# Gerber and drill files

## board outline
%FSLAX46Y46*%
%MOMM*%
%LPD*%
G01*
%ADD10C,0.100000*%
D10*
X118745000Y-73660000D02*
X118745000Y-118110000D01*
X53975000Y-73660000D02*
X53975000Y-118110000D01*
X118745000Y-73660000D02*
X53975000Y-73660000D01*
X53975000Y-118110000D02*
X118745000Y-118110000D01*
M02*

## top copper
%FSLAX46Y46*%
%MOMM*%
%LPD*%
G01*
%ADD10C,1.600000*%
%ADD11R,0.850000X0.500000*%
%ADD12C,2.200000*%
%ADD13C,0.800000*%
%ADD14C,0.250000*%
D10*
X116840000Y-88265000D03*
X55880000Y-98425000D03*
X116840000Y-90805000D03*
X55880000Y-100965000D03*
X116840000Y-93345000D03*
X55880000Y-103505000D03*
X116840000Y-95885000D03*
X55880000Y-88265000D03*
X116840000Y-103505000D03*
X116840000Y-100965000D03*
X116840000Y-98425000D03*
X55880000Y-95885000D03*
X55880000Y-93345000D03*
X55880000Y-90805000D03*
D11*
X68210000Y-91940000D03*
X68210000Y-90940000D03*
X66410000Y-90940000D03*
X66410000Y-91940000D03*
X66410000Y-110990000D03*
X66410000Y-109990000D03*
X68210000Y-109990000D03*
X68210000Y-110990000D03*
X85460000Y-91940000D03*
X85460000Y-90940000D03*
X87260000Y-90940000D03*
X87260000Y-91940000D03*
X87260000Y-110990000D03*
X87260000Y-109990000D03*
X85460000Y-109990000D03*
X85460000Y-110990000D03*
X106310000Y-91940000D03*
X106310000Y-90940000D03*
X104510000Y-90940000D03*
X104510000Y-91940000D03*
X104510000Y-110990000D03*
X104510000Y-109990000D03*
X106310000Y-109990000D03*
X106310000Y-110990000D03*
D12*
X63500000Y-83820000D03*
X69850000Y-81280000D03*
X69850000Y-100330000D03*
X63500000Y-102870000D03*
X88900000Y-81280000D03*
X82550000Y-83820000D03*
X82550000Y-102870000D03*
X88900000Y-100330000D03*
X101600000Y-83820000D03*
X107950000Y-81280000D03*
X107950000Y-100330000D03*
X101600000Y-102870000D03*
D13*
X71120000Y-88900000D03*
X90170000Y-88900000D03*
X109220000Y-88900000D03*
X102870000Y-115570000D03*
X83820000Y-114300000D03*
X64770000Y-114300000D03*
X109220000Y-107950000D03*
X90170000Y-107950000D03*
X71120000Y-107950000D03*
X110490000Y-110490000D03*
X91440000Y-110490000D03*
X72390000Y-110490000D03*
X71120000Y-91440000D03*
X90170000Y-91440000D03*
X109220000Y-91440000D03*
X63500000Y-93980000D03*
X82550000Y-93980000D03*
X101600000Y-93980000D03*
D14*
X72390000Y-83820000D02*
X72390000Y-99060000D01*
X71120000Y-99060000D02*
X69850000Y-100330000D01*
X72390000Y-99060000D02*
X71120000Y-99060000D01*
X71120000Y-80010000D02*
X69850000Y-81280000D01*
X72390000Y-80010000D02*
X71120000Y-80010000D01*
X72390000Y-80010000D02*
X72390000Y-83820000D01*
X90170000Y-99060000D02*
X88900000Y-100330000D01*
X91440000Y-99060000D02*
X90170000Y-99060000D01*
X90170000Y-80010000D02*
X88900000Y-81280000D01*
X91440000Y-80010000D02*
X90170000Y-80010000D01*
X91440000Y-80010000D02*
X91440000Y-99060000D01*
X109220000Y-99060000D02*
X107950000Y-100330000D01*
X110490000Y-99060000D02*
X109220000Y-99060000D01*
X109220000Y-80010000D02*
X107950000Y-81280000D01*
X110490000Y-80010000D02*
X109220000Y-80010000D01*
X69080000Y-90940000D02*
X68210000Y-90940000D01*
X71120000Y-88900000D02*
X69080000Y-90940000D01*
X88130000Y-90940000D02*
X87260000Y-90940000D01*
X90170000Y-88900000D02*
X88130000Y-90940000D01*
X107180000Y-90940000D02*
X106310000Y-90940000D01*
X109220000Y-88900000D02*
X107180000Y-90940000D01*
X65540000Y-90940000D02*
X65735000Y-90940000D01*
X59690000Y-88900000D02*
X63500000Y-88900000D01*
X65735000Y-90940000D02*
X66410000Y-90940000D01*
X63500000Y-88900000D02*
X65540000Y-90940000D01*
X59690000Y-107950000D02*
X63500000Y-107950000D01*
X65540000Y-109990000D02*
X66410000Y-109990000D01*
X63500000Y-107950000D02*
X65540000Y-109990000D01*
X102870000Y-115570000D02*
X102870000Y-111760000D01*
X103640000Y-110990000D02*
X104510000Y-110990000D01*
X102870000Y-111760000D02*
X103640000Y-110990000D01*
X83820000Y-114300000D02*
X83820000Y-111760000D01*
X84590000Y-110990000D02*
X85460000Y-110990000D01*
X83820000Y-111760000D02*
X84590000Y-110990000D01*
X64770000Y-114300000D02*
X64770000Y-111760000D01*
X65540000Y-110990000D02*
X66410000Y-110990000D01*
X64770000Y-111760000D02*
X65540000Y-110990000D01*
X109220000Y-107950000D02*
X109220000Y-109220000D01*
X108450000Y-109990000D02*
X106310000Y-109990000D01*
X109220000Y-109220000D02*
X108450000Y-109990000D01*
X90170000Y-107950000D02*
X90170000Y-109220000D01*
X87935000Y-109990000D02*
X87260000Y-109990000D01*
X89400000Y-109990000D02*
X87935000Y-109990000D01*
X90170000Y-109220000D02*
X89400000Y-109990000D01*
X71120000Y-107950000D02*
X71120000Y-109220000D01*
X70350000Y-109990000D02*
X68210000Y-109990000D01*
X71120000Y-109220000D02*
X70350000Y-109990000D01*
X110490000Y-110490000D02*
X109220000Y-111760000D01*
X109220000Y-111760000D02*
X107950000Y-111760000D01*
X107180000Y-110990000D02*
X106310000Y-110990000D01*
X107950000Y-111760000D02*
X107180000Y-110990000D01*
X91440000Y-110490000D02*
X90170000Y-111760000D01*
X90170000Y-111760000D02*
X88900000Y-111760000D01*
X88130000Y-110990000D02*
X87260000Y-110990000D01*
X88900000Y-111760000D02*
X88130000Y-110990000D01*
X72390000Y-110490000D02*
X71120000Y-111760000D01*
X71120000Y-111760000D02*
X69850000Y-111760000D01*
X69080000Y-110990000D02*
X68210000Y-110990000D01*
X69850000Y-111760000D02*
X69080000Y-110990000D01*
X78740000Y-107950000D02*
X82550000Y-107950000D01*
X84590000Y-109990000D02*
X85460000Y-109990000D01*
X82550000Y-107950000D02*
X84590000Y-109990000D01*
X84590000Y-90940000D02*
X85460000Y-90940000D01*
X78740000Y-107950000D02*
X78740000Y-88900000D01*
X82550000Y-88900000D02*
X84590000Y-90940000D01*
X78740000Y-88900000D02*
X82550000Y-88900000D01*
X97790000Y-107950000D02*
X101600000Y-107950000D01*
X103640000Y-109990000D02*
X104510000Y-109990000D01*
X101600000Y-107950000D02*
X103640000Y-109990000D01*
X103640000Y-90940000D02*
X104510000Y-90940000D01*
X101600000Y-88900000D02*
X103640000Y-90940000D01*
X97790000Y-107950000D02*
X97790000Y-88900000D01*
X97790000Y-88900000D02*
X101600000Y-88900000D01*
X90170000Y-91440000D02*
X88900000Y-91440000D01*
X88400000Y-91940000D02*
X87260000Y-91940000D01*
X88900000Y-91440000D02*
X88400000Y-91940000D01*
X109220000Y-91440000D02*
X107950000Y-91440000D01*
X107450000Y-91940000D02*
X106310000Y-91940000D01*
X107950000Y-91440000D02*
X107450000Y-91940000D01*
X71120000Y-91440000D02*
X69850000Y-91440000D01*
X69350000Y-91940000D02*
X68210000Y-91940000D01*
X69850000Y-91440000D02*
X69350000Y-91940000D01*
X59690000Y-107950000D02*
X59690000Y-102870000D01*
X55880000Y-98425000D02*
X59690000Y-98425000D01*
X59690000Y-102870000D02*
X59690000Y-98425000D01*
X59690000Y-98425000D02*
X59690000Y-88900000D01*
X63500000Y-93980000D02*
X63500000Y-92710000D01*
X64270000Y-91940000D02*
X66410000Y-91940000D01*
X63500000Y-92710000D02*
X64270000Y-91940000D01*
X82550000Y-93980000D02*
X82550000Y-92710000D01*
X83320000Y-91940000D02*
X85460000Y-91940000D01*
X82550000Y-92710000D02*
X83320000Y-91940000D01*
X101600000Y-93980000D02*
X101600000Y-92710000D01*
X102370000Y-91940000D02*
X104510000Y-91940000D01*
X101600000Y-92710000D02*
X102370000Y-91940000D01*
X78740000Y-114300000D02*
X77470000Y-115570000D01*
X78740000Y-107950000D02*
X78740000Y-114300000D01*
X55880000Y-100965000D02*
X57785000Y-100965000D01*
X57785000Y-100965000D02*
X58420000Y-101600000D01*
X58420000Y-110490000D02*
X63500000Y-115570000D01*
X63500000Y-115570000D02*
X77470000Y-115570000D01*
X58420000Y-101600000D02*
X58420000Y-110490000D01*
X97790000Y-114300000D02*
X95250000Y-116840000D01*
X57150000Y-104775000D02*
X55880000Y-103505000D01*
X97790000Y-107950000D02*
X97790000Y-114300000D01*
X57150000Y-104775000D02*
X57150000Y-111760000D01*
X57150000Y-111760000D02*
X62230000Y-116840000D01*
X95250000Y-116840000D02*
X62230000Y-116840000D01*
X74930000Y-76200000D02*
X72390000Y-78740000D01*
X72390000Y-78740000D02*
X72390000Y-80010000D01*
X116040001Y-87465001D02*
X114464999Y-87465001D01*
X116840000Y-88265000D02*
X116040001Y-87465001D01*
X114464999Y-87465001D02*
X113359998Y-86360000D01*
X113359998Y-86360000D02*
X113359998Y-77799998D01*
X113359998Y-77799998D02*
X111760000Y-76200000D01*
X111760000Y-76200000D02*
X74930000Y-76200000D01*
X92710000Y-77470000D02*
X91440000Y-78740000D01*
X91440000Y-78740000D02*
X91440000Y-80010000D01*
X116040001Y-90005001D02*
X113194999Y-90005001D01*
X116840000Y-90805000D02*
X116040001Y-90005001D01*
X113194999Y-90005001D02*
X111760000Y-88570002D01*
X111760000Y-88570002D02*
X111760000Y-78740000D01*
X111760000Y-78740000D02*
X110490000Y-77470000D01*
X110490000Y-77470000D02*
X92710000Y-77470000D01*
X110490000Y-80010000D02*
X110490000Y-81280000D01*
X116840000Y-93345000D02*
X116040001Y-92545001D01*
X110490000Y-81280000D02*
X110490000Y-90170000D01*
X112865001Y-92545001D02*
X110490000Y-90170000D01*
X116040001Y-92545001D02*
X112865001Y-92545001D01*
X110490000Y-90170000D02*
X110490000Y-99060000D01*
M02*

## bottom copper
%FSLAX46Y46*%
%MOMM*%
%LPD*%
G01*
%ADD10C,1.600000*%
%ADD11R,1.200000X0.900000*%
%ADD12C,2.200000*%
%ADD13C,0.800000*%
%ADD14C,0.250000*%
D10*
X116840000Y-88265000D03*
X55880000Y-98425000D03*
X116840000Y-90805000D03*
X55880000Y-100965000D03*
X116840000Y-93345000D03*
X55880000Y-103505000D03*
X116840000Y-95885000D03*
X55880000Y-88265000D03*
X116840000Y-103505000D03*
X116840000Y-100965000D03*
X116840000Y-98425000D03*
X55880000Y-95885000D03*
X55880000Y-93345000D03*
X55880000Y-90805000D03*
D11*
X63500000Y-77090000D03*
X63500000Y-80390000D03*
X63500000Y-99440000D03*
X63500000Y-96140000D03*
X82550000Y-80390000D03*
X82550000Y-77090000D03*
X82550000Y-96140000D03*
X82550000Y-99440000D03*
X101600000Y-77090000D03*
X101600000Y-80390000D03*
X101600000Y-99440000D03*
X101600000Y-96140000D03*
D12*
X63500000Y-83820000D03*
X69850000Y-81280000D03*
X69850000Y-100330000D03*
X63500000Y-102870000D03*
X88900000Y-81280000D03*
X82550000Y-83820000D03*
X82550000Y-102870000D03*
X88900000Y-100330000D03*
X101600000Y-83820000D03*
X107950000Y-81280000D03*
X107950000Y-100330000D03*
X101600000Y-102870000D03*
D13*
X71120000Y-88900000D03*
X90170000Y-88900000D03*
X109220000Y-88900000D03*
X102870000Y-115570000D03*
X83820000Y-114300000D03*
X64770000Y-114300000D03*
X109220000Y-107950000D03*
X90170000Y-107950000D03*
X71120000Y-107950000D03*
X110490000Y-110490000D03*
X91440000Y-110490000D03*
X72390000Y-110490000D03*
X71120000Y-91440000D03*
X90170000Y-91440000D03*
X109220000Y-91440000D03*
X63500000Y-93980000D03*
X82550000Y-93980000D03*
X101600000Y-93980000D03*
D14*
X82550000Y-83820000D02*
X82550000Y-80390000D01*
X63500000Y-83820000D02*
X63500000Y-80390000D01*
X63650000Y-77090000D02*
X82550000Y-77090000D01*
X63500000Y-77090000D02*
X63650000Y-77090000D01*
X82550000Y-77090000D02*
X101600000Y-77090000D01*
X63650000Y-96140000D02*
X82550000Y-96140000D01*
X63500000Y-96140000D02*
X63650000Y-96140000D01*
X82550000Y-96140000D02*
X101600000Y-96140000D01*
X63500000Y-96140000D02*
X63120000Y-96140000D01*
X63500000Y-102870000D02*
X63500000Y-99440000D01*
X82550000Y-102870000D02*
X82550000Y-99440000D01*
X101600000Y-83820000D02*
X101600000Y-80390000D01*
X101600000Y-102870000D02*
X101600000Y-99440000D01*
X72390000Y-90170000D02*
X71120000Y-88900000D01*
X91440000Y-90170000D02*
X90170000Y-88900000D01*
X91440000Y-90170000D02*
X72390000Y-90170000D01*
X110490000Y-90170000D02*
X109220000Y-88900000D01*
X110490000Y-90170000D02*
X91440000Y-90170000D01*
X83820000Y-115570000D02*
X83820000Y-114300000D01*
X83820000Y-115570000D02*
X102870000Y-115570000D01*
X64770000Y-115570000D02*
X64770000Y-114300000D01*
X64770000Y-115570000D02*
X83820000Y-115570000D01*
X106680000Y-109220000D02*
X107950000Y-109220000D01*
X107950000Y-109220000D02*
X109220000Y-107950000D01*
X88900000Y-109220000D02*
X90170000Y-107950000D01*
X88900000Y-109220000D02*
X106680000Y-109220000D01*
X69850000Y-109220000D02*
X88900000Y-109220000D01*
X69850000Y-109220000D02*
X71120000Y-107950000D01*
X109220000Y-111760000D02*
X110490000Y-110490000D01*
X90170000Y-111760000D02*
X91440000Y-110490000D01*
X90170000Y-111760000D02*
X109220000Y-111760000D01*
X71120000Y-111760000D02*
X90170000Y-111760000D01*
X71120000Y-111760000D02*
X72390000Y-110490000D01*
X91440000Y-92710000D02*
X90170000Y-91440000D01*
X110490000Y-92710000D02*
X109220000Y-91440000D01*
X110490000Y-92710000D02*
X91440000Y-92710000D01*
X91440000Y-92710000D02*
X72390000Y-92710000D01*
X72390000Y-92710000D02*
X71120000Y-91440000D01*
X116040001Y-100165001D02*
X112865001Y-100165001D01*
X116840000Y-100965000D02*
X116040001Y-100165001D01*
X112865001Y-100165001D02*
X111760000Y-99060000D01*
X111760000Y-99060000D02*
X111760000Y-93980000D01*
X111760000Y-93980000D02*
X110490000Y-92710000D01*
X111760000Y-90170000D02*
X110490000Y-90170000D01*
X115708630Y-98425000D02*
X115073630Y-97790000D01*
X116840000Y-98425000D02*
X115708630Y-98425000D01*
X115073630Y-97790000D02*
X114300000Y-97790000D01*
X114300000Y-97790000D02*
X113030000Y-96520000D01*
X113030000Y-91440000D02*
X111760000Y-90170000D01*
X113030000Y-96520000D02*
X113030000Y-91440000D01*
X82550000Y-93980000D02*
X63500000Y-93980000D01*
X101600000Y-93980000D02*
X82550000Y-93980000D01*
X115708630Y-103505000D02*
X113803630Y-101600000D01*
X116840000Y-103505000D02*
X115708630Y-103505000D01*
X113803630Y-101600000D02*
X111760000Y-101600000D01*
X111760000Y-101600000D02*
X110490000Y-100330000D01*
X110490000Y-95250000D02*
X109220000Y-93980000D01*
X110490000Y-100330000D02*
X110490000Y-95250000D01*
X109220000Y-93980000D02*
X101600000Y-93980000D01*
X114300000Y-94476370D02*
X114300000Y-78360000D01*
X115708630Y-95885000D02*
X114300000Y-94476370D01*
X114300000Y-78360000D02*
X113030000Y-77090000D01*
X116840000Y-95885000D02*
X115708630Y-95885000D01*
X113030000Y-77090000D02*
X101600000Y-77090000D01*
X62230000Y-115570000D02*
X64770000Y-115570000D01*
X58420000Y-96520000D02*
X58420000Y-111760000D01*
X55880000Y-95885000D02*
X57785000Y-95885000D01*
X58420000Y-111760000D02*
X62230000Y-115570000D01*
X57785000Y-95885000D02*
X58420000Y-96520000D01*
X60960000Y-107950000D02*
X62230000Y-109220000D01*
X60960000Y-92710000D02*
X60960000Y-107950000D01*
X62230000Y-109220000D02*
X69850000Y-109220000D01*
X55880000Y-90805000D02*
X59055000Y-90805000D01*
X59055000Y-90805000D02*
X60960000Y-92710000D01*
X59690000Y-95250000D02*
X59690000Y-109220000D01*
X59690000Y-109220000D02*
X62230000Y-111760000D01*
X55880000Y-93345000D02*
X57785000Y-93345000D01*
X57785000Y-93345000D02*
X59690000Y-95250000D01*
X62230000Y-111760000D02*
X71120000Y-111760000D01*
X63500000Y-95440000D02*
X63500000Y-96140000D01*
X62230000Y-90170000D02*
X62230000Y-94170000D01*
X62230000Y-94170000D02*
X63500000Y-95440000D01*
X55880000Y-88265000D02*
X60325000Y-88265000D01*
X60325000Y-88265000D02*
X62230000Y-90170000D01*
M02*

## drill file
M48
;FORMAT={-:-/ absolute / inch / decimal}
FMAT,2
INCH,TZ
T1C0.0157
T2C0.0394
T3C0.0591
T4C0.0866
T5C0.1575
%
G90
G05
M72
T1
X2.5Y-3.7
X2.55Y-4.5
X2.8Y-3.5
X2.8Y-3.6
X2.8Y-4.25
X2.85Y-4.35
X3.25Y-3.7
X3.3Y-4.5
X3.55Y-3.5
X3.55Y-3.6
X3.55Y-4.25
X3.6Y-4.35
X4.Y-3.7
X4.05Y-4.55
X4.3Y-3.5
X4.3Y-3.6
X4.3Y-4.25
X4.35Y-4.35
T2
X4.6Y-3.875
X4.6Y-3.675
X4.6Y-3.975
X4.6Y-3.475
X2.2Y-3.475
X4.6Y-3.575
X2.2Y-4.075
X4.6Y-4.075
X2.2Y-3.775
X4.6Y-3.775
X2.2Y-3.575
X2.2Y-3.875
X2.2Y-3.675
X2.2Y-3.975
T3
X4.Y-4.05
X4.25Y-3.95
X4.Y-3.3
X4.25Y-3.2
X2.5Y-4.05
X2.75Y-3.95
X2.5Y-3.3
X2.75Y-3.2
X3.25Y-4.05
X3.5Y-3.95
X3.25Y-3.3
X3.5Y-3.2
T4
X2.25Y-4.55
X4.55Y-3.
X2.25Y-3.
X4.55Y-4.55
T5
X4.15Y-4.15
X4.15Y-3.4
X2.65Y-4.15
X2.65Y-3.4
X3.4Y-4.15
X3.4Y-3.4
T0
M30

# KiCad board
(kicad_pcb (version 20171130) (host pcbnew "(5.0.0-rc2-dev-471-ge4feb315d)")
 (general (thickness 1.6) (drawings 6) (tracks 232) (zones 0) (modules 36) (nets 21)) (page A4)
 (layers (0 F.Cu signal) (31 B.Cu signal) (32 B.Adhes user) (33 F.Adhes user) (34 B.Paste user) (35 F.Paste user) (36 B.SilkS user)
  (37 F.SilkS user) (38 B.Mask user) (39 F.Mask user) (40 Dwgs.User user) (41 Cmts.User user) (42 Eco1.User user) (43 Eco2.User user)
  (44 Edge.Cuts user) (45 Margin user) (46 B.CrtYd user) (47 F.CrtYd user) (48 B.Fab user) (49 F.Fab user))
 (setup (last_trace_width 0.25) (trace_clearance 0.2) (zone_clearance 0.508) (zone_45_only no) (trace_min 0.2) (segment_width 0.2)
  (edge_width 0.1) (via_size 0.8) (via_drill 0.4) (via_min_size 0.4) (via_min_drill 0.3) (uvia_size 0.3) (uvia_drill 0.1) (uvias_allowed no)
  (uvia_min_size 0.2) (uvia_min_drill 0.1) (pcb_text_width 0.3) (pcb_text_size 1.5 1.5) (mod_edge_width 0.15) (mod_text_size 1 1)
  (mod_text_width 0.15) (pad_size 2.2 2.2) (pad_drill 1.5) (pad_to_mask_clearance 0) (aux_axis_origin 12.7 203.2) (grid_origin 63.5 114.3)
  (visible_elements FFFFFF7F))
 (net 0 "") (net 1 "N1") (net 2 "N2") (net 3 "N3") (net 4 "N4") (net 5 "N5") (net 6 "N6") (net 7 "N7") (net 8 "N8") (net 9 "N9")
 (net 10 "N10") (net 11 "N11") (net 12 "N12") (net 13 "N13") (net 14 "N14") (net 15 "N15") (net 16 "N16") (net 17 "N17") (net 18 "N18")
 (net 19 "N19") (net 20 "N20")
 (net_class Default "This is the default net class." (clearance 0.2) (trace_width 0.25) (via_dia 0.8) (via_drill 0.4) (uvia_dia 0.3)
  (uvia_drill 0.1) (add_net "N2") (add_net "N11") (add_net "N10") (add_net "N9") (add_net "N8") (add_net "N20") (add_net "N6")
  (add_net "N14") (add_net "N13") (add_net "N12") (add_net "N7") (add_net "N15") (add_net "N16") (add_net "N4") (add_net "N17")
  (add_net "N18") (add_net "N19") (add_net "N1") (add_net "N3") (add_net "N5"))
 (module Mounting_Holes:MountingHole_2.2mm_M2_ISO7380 (layer F.Cu) (at 115.57 76.2)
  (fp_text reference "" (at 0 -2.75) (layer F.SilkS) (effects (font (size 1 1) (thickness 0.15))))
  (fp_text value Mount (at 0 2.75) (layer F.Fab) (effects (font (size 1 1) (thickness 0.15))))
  (pad 1 np_thru_hole circle (at 0 0) (size 2.2 2.2) (drill 2.2) (layers *.Cu *.Mask)))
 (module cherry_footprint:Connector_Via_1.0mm (layer F.Cu) (at 116.84 88.265 90)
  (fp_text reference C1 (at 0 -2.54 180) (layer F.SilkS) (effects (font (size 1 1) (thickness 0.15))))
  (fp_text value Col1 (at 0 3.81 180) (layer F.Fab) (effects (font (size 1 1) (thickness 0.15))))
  (pad 1 thru_hole circle (at 0 0 90) (size 1.6 1.6) (drill 1) (layers *.Cu *.Mask) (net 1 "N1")))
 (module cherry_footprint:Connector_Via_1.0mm (layer F.Cu) (at 55.88 98.425 270)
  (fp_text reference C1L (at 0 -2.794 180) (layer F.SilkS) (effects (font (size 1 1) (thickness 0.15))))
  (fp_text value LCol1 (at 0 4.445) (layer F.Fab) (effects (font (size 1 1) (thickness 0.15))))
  (pad 1 thru_hole circle (at 0 0 270) (size 1.6 1.6) (drill 1) (layers *.Cu *.Mask) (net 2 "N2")))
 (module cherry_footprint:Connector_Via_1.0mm (layer F.Cu) (at 116.84 90.805 90)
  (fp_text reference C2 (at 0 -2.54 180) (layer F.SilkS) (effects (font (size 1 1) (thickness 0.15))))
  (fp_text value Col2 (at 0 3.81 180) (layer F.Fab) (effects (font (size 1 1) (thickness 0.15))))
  (pad 1 thru_hole circle (at 0 0 90) (size 1.6 1.6) (drill 1) (layers *.Cu *.Mask) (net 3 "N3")))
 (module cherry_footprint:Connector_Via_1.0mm (layer F.Cu) (at 55.88 100.965 270)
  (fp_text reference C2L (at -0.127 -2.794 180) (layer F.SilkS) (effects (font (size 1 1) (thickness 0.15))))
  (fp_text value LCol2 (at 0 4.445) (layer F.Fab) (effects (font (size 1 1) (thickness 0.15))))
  (pad 1 thru_hole circle (at 0 0 270) (size 1.6 1.6) (drill 1) (layers *.Cu *.Mask) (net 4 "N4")))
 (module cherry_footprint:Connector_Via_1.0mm (layer F.Cu) (at 116.84 93.345 90)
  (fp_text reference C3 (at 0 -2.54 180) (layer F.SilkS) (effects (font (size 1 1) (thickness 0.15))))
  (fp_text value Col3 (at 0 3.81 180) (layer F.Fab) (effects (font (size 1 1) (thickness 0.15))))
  (pad 1 thru_hole circle (at 0 0 90) (size 1.6 1.6) (drill 1) (layers *.Cu *.Mask) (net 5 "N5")))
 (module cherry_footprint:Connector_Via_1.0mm (layer F.Cu) (at 55.88 103.505 270)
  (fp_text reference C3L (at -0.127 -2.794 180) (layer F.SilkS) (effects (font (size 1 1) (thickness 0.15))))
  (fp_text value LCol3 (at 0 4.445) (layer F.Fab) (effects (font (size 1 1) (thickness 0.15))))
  (pad 1 thru_hole circle (at 0 0 270) (size 1.6 1.6) (drill 1) (layers *.Cu *.Mask) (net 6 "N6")))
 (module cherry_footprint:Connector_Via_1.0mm (layer F.Cu) (at 116.84 95.885 90)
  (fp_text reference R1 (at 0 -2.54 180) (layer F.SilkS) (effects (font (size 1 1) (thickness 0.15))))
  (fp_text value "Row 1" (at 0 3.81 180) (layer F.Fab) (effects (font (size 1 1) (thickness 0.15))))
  (pad 1 thru_hole circle (at 0 0 90) (size 1.6 1.6) (drill 1) (layers *.Cu *.Mask) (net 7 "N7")))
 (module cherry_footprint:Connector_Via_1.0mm (layer F.Cu) (at 55.88 88.265 270)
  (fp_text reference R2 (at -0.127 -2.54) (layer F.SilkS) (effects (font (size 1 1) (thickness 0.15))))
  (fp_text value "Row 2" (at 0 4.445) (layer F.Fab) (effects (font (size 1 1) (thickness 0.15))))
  (pad 1 thru_hole circle (at 0 0 270) (size 1.6 1.6) (drill 1) (layers *.Cu *.Mask) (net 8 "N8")))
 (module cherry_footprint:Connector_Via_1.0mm (layer F.Cu) (at 116.84 103.505 90)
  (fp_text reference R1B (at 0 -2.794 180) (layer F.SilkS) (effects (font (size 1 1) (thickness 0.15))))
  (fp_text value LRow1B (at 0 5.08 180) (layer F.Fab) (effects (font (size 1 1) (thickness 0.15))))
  (pad 1 thru_hole circle (at 0 0 90) (size 1.6 1.6) (drill 1) (layers *.Cu *.Mask) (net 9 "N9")))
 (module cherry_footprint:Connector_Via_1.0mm (layer F.Cu) (at 116.84 100.965 90)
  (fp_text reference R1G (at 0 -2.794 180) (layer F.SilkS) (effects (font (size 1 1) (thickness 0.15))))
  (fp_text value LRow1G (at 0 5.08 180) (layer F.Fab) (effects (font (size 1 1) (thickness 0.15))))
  (pad 1 thru_hole circle (at 0 0 90) (size 1.6 1.6) (drill 1) (layers *.Cu *.Mask) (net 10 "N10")))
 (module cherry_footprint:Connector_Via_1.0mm (layer F.Cu) (at 116.84 98.425 90)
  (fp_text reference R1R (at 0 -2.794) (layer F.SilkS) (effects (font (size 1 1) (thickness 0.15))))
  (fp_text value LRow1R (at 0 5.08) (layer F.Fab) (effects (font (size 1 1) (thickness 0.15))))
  (pad 1 thru_hole circle (at 0 0 90) (size 1.6 1.6) (drill 1) (layers *.Cu *.Mask) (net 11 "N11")))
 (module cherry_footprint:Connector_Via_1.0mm (layer F.Cu) (at 55.88 95.885 270)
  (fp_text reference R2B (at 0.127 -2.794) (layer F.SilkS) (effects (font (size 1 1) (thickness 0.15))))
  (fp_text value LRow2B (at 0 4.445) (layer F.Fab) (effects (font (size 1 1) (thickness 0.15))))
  (pad 1 thru_hole circle (at 0 0 270) (size 1.6 1.6) (drill 1) (layers *.Cu *.Mask) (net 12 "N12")))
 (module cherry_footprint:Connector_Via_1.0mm (layer F.Cu) (at 55.88 93.345 270)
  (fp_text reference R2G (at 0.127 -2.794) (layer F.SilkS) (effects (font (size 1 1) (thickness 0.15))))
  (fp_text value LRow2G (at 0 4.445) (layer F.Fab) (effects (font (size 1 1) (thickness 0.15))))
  (pad 1 thru_hole circle (at 0 0 270) (size 1.6 1.6) (drill 1) (layers *.Cu *.Mask) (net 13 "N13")))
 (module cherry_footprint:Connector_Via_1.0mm (layer F.Cu) (at 55.88 90.805 270)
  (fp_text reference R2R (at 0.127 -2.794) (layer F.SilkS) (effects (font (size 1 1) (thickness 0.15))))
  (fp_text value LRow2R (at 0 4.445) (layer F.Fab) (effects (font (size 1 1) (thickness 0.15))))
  (pad 1 thru_hole circle (at 0 0 270) (size 1.6 1.6) (drill 1) (layers *.Cu *.Mask) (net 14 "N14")))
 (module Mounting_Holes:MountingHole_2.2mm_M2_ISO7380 (layer F.Cu) (at 57.15 115.57)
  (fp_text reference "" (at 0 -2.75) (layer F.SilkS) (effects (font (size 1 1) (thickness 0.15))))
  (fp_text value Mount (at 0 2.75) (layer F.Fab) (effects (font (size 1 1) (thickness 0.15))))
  (pad 1 np_thru_hole circle (at 0 0) (size 2.2 2.2) (drill 2.2) (layers *.Cu *.Mask)))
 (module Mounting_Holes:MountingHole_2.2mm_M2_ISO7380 (layer F.Cu) (at 115.57 115.57)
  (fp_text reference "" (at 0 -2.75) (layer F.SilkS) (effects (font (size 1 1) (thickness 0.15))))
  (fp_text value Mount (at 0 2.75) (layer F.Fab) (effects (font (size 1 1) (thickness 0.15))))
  (pad 1 np_thru_hole circle (at 0 0) (size 2.2 2.2) (drill 2.2) (layers *.Cu *.Mask)))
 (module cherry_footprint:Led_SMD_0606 (layer F.Cu) (at 67.31 91.44 180)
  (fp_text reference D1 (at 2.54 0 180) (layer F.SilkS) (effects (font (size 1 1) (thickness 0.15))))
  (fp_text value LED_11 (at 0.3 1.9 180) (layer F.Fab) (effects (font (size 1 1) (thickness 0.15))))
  (pad 3 smd rect (at -0.9 -0.5 180) (size 0.85 0.5) (layers F.Cu F.Paste F.Mask) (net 10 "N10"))
  (pad 2 smd rect (at -0.9 0.5 180) (size 0.85 0.5) (layers F.Cu F.Paste F.Mask) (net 11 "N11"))
  (pad 1 smd rect (at 0.9 0.5 180) (size 0.85 0.5) (layers F.Cu F.Paste F.Mask) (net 2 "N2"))
  (pad 4 smd rect (at 0.9 -0.5 180) (size 0.85 0.5) (layers F.Cu F.Paste F.Mask) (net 9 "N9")))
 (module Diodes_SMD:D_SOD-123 (layer B.Cu) (at 63.5 78.74 270)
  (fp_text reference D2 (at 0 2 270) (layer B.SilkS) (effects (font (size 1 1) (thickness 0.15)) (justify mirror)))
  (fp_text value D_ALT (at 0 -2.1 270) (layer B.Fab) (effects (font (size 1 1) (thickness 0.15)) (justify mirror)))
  (pad 1 smd rect (at -1.65 0 270) (size 0.9 1.2) (layers B.Cu B.Paste B.Mask) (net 7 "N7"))
  (pad 2 smd rect (at 1.65 0 270) (size 0.9 1.2) (layers B.Cu B.Paste B.Mask) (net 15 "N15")))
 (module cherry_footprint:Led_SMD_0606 (layer F.Cu) (at 67.31 110.49 180)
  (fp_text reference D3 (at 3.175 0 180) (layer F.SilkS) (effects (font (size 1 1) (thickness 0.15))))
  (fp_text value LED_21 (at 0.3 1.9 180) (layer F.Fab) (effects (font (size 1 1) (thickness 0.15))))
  (pad 4 smd rect (at 0.9 -0.5 180) (size 0.85 0.5) (layers F.Cu F.Paste F.Mask) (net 12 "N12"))
  (pad 1 smd rect (at 0.9 0.5 180) (size 0.85 0.5) (layers F.Cu F.Paste F.Mask) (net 2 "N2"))
  (pad 2 smd rect (at -0.9 0.5 180) (size 0.85 0.5) (layers F.Cu F.Paste F.Mask) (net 14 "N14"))
  (pad 3 smd rect (at -0.9 -0.5 180) (size 0.85 0.5) (layers F.Cu F.Paste F.Mask) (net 13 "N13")))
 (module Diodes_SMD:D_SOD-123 (layer B.Cu) (at 63.5 97.79 270)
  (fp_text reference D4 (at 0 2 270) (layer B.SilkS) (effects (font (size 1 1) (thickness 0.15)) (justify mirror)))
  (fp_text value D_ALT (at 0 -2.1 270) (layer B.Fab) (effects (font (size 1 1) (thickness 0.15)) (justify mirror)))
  (pad 2 smd rect (at 1.65 0 270) (size 0.9 1.2) (layers B.Cu B.Paste B.Mask) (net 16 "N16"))
  (pad 1 smd rect (at -1.65 0 270) (size 0.9 1.2) (layers B.Cu B.Paste B.Mask) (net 8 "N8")))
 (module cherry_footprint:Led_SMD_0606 (layer F.Cu) (at 86.36 91.44 180)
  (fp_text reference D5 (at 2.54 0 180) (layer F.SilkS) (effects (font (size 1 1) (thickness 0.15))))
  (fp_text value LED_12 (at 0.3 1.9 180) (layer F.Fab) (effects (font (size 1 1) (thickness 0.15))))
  (pad 4 smd rect (at 0.9 -0.5 180) (size 0.85 0.5) (layers F.Cu F.Paste F.Mask) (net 9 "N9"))
  (pad 1 smd rect (at 0.9 0.5 180) (size 0.85 0.5) (layers F.Cu F.Paste F.Mask) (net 4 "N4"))
  (pad 2 smd rect (at -0.9 0.5 180) (size 0.85 0.5) (layers F.Cu F.Paste F.Mask) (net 11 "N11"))
  (pad 3 smd rect (at -0.9 -0.5 180) (size 0.85 0.5) (layers F.Cu F.Paste F.Mask) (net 10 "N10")))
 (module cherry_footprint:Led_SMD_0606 (layer F.Cu) (at 86.36 110.49 180)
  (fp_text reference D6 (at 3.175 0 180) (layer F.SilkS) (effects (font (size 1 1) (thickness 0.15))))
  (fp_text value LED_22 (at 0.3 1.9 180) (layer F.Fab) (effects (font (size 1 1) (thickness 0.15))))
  (pad 3 smd rect (at -0.9 -0.5 180) (size 0.85 0.5) (layers F.Cu F.Paste F.Mask) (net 13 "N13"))
  (pad 2 smd rect (at -0.9 0.5 180) (size 0.85 0.5) (layers F.Cu F.Paste F.Mask) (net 14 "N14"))
  (pad 1 smd rect (at 0.9 0.5 180) (size 0.85 0.5) (layers F.Cu F.Paste F.Mask) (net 4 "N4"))
  (pad 4 smd rect (at 0.9 -0.5 180) (size 0.85 0.5) (layers F.Cu F.Paste F.Mask) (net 12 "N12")))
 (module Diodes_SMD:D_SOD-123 (layer B.Cu) (at 82.55 78.74 270)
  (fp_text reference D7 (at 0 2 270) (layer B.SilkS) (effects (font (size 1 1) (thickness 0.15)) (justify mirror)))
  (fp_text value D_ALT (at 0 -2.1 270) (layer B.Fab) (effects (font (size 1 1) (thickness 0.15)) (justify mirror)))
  (pad 2 smd rect (at 1.65 0 270) (size 0.9 1.2) (layers B.Cu B.Paste B.Mask) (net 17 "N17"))
  (pad 1 smd rect (at -1.65 0 270) (size 0.9 1.2) (layers B.Cu B.Paste B.Mask) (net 7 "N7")))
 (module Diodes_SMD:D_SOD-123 (layer B.Cu) (at 82.55 97.79 270)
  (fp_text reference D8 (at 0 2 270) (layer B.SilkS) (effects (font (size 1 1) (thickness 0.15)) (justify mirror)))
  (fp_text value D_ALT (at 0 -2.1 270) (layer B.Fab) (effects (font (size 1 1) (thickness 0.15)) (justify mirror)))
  (pad 1 smd rect (at -1.65 0 270) (size 0.9 1.2) (layers B.Cu B.Paste B.Mask) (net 8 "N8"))
  (pad 2 smd rect (at 1.65 0 270) (size 0.9 1.2) (layers B.Cu B.Paste B.Mask) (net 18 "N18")))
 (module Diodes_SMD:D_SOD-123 (layer B.Cu) (at 101.6 78.74 270)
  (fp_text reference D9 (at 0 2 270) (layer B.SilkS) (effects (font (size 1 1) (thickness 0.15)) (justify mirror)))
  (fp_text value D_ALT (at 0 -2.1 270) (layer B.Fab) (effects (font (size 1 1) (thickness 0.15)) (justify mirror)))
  (pad 1 smd rect (at -1.65 0 270) (size 0.9 1.2) (layers B.Cu B.Paste B.Mask) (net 7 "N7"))
  (pad 2 smd rect (at 1.65 0 270) (size 0.9 1.2) (layers B.Cu B.Paste B.Mask) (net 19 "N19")))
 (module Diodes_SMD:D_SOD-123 (layer B.Cu) (at 101.6 97.79 270)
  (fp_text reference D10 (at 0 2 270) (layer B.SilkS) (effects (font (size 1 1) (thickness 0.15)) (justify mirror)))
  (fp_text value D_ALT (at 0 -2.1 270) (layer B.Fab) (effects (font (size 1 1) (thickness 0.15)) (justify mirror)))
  (pad 2 smd rect (at 1.65 0 270) (size 0.9 1.2) (layers B.Cu B.Paste B.Mask) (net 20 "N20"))
  (pad 1 smd rect (at -1.65 0 270) (size 0.9 1.2) (layers B.Cu B.Paste B.Mask) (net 8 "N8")))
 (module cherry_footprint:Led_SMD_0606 (layer F.Cu) (at 105.41 91.44 180)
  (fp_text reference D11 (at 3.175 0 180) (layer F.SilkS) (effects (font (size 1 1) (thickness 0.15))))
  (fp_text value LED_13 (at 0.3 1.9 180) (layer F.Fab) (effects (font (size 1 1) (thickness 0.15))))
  (pad 3 smd rect (at -0.9 -0.5 180) (size 0.85 0.5) (layers F.Cu F.Paste F.Mask) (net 10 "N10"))
  (pad 2 smd rect (at -0.9 0.5 180) (size 0.85 0.5) (layers F.Cu F.Paste F.Mask) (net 11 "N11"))
  (pad 1 smd rect (at 0.9 0.5 180) (size 0.85 0.5) (layers F.Cu F.Paste F.Mask) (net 6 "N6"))
  (pad 4 smd rect (at 0.9 -0.5 180) (size 0.85 0.5) (layers F.Cu F.Paste F.Mask) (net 9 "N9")))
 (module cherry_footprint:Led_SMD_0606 (layer F.Cu) (at 105.41 110.49 180)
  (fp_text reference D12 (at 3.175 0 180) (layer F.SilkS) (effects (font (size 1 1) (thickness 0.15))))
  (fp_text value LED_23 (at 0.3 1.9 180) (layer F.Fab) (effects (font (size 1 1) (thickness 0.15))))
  (pad 4 smd rect (at 0.9 -0.5 180) (size 0.85 0.5) (layers F.Cu F.Paste F.Mask) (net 12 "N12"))
  (pad 1 smd rect (at 0.9 0.5 180) (size 0.85 0.5) (layers F.Cu F.Paste F.Mask) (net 6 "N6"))
  (pad 2 smd rect (at -0.9 0.5 180) (size 0.85 0.5) (layers F.Cu F.Paste F.Mask) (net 14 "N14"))
  (pad 3 smd rect (at -0.9 -0.5 180) (size 0.85 0.5) (layers F.Cu F.Paste F.Mask) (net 13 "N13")))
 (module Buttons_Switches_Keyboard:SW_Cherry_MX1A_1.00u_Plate (layer F.Cu) (at 69.85 81.28)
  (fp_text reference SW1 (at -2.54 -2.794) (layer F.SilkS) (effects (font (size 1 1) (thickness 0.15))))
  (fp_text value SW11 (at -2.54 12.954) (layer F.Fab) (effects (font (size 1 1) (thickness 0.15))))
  (pad "" np_thru_hole circle (at -2.54 5.08) (size 4 4) (drill 4) (layers *.Cu *.Mask))
  (pad 2 thru_hole circle (at -6.35 2.54) (size 2.2 2.2) (drill 1.5) (layers *.Cu *.Mask) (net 15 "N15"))
  (pad 1 thru_hole circle (at 0 0) (size 2.2 2.2) (drill 1.5) (layers *.Cu *.Mask) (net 1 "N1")))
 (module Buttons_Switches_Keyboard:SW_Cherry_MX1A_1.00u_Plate (layer F.Cu) (at 69.85 100.33)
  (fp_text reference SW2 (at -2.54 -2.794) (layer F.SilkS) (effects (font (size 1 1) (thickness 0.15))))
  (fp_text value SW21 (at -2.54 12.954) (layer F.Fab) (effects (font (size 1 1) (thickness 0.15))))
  (pad 1 thru_hole circle (at 0 0) (size 2.2 2.2) (drill 1.5) (layers *.Cu *.Mask) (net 1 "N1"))
  (pad 2 thru_hole circle (at -6.35 2.54) (size 2.2 2.2) (drill 1.5) (layers *.Cu *.Mask) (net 16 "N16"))
  (pad "" np_thru_hole circle (at -2.54 5.08) (size 4 4) (drill 4) (layers *.Cu *.Mask)))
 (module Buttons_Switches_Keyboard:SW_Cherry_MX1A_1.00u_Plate (layer F.Cu) (at 88.9 81.28)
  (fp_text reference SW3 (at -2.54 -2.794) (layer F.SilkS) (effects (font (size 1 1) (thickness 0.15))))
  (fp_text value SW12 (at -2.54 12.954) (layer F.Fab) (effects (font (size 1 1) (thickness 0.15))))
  (pad 1 thru_hole circle (at 0 0) (size 2.2 2.2) (drill 1.5) (layers *.Cu *.Mask) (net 3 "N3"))
  (pad 2 thru_hole circle (at -6.35 2.54) (size 2.2 2.2) (drill 1.5) (layers *.Cu *.Mask) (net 17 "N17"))
  (pad "" np_thru_hole circle (at -2.54 5.08) (size 4 4) (drill 4) (layers *.Cu *.Mask)))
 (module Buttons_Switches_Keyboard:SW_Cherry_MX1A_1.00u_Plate (layer F.Cu) (at 88.9 100.33)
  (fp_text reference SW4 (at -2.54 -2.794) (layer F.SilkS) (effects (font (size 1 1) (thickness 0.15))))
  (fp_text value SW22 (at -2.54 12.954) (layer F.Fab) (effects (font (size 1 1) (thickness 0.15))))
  (pad "" np_thru_hole circle (at -2.54 5.08) (size 4 4) (drill 4) (layers *.Cu *.Mask))
  (pad 2 thru_hole circle (at -6.35 2.54) (size 2.2 2.2) (drill 1.5) (layers *.Cu *.Mask) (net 18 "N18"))
  (pad 1 thru_hole circle (at 0 0) (size 2.2 2.2) (drill 1.5) (layers *.Cu *.Mask) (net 3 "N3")))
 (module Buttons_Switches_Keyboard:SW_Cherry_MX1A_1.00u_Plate (layer F.Cu) (at 107.95 81.28)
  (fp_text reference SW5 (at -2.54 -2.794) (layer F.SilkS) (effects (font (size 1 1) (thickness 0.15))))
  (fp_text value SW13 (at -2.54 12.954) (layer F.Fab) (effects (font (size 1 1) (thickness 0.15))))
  (pad "" np_thru_hole circle (at -2.54 5.08) (size 4 4) (drill 4) (layers *.Cu *.Mask))
  (pad 2 thru_hole circle (at -6.35 2.54) (size 2.2 2.2) (drill 1.5) (layers *.Cu *.Mask) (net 19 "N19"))
  (pad 1 thru_hole circle (at 0 0) (size 2.2 2.2) (drill 1.5) (layers *.Cu *.Mask) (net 5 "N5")))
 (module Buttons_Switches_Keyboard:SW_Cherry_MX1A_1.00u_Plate (layer F.Cu) (at 107.95 100.33)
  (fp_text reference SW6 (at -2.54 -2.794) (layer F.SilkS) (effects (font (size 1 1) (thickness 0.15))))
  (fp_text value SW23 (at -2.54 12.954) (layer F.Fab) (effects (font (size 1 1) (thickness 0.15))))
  (pad 1 thru_hole circle (at 0 0) (size 2.2 2.2) (drill 1.5) (layers *.Cu *.Mask) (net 5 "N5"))
  (pad 2 thru_hole circle (at -6.35 2.54) (size 2.2 2.2) (drill 1.5) (layers *.Cu *.Mask) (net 20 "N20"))
  (pad "" np_thru_hole circle (at -2.54 5.08) (size 4 4) (drill 4) (layers *.Cu *.Mask)))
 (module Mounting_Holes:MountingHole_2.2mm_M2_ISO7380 (layer F.Cu) (at 57.15 76.2)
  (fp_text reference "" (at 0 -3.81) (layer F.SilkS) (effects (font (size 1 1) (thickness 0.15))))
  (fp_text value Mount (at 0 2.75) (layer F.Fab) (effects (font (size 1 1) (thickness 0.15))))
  (pad 1 np_thru_hole circle (at 0 0) (size 2.2 2.2) (drill 2.2) (layers *.Cu *.Mask)))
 (gr_line (start 118.745 73.66) (end 118.745 118.11) (layer Edge.Cuts) (width 0.1))
 (gr_line (start 53.975 73.66) (end 53.975 118.11) (layer Edge.Cuts) (width 0.1))
 (gr_line (start 118.745 73.66) (end 53.975 73.66) (layer Edge.Cuts) (width 0.1))
 (gr_line (start 53.975 118.11) (end 118.745 118.11) (layer Edge.Cuts) (width 0.1))
 (segment (start 72.39 83.82) (end 72.39 99.06) (width 0.25) (layer F.Cu) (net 1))
 (segment (start 71.12 99.06) (end 69.85 100.33) (width 0.25) (layer F.Cu) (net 1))
 (segment (start 72.39 99.06) (end 71.12 99.06) (width 0.25) (layer F.Cu) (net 1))
 (segment (start 71.12 80.01) (end 69.85 81.28) (width 0.25) (layer F.Cu) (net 1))
 (segment (start 72.39 80.01) (end 71.12 80.01) (width 0.25) (layer F.Cu) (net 1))
 (segment (start 72.39 80.01) (end 72.39 83.82) (width 0.25) (layer F.Cu) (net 1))
 (segment (start 90.17 99.06) (end 88.9 100.33) (width 0.25) (layer F.Cu) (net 3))
 (segment (start 91.44 99.06) (end 90.17 99.06) (width 0.25) (layer F.Cu) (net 3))
 (segment (start 90.17 80.01) (end 88.9 81.28) (width 0.25) (layer F.Cu) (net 3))
 (segment (start 91.44 80.01) (end 90.17 80.01) (width 0.25) (layer F.Cu) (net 3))
 (segment (start 91.44 80.01) (end 91.44 99.06) (width 0.25) (layer F.Cu) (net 3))
 (segment (start 109.22 99.06) (end 107.95 100.33) (width 0.25) (layer F.Cu) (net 5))
 (segment (start 110.49 99.06) (end 109.22 99.06) (width 0.25) (layer F.Cu) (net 5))
 (segment (start 109.22 80.01) (end 107.95 81.28) (width 0.25) (layer F.Cu) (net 5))
 (segment (start 110.49 80.01) (end 109.22 80.01) (width 0.25) (layer F.Cu) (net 5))
 (segment (start 82.55 83.82) (end 82.55 80.39) (width 0.25) (layer B.Cu) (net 17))
 (segment (start 63.5 83.82) (end 63.5 80.39) (width 0.25) (layer B.Cu) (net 15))
 (segment (start 63.65 77.09) (end 82.55 77.09) (width 0.25) (layer B.Cu) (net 7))
 (segment (start 63.5 77.09) (end 63.65 77.09) (width 0.25) (layer B.Cu) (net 7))
 (segment (start 82.55 77.09) (end 101.6 77.09) (width 0.25) (layer B.Cu) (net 7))
 (segment (start 63.65 96.14) (end 82.55 96.14) (width 0.25) (layer B.Cu) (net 8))
 (segment (start 63.5 96.14) (end 63.65 96.14) (width 0.25) (layer B.Cu) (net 8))
 (segment (start 82.55 96.14) (end 101.6 96.14) (width 0.25) (layer B.Cu) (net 8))
 (segment (start 63.5 96.14) (end 63.12 96.14) (width 0.25) (layer B.Cu) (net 8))
 (segment (start 63.5 102.87) (end 63.5 99.44) (width 0.25) (layer B.Cu) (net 16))
 (segment (start 82.55 102.87) (end 82.55 99.44) (width 0.25) (layer B.Cu) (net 18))
 (segment (start 101.6 83.82) (end 101.6 80.39) (width 0.25) (layer B.Cu) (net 19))
 (segment (start 101.6 102.87) (end 101.6 99.44) (width 0.25) (layer B.Cu) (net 20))
 (via (at 71.12 88.9) (size 0.8) (drill 0.4) (layers F.Cu B.Cu) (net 11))
 (segment (start 72.39 90.17) (end 71.12 88.9) (width 0.25) (layer B.Cu) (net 11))
 (segment (start 69.08 90.94) (end 68.21 90.94) (width 0.25) (layer F.Cu) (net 11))
 (segment (start 71.12 88.9) (end 69.08 90.94) (width 0.25) (layer F.Cu) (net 11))
 (segment (start 91.44 90.17) (end 90.17 88.9) (width 0.25) (layer B.Cu) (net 11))
 (segment (start 91.44 90.17) (end 72.39 90.17) (width 0.25) (layer B.Cu) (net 11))
 (via (at 90.17 88.9) (size 0.8) (drill 0.4) (layers F.Cu B.Cu) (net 11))
 (segment (start 88.13 90.94) (end 87.26 90.94) (width 0.25) (layer F.Cu) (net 11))
 (segment (start 90.17 88.9) (end 88.13 90.94) (width 0.25) (layer F.Cu) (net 11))
 (segment (start 110.49 90.17) (end 109.22 88.9) (width 0.25) (layer B.Cu) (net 11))
 (segment (start 110.49 90.17) (end 91.44 90.17) (width 0.25) (layer B.Cu) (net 11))
 (via (at 109.22 88.9) (size 0.8) (drill 0.4) (layers F.Cu B.Cu) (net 11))
 (segment (start 107.18 90.94) (end 106.31 90.94) (width 0.25) (layer F.Cu) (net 11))
 (segment (start 109.22 88.9) (end 107.18 90.94) (width 0.25) (layer F.Cu) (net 11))
 (segment (start 65.54 90.94) (end 65.735 90.94) (width 0.25) (layer F.Cu) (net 2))
 (segment (start 59.69 88.9) (end 63.5 88.9) (width 0.25) (layer F.Cu) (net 2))
 (segment (start 65.735 90.94) (end 66.41 90.94) (width 0.25) (layer F.Cu) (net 2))
 (segment (start 63.5 88.9) (end 65.54 90.94) (width 0.25) (layer F.Cu) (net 2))
 (segment (start 59.69 107.95) (end 63.5 107.95) (width 0.25) (layer F.Cu) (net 2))
 (segment (start 65.54 109.99) (end 66.41 109.99) (width 0.25) (layer F.Cu) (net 2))
 (segment (start 63.5 107.95) (end 65.54 109.99) (width 0.25) (layer F.Cu) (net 2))
 (via (at 102.87 115.57) (size 0.8) (drill 0.4) (layers F.Cu B.Cu) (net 12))
 (segment (start 102.87 115.57) (end 102.87 111.76) (width 0.25) (layer F.Cu) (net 12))
 (segment (start 103.64 110.99) (end 104.51 110.99) (width 0.25) (layer F.Cu) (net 12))
 (segment (start 102.87 111.76) (end 103.64 110.99) (width 0.25) (layer F.Cu) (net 12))
 (via (at 83.82 114.3) (size 0.8) (drill 0.4) (layers F.Cu B.Cu) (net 12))
 (segment (start 83.82 115.57) (end 83.82 114.3) (width 0.25) (layer B.Cu) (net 12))
 (segment (start 83.82 115.57) (end 102.87 115.57) (width 0.25) (layer B.Cu) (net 12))
 (segment (start 83.82 114.3) (end 83.82 111.76) (width 0.25) (layer F.Cu) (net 12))
 (segment (start 84.59 110.99) (end 85.46 110.99) (width 0.25) (layer F.Cu) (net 12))
 (segment (start 83.82 111.76) (end 84.59 110.99) (width 0.25) (layer F.Cu) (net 12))
 (via (at 64.77 114.3) (size 0.8) (drill 0.4) (layers F.Cu B.Cu) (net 12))
 (segment (start 64.77 115.57) (end 64.77 114.3) (width 0.25) (layer B.Cu) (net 12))
 (segment (start 64.77 115.57) (end 83.82 115.57) (width 0.25) (layer B.Cu) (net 12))
 (segment (start 64.77 114.3) (end 64.77 111.76) (width 0.25) (layer F.Cu) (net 12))
 (segment (start 65.54 110.99) (end 66.41 110.99) (width 0.25) (layer F.Cu) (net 12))
 (segment (start 64.77 111.76) (end 65.54 110.99) (width 0.25) (layer F.Cu) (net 12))
 (via (at 109.22 107.95) (size 0.8) (drill 0.4) (layers F.Cu B.Cu) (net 14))
 (segment (start 106.68 109.22) (end 107.95 109.22) (width 0.25) (layer B.Cu) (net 14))
 (segment (start 107.95 109.22) (end 109.22 107.95) (width 0.25) (layer B.Cu) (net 14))
 (segment (start 109.22 107.95) (end 109.22 109.22) (width 0.25) (layer F.Cu) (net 14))
 (segment (start 108.45 109.99) (end 106.31 109.99) (width 0.25) (layer F.Cu) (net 14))
 (segment (start 109.22 109.22) (end 108.45 109.99) (width 0.25) (layer F.Cu) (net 14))
 (via (at 90.17 107.95) (size 0.8) (drill 0.4) (layers F.Cu B.Cu) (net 14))
 (segment (start 88.9 109.22) (end 90.17 107.95) (width 0.25) (layer B.Cu) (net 14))
 (segment (start 88.9 109.22) (end 106.68 109.22) (width 0.25) (layer B.Cu) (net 14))
 (segment (start 90.17 107.95) (end 90.17 109.22) (width 0.25) (layer F.Cu) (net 14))
 (segment (start 87.935 109.99) (end 87.26 109.99) (width 0.25) (layer F.Cu) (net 14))
 (segment (start 89.4 109.99) (end 87.935 109.99) (width 0.25) (layer F.Cu) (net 14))
 (segment (start 90.17 109.22) (end 89.4 109.99) (width 0.25) (layer F.Cu) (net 14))
 (via (at 71.12 107.95) (size 0.8) (drill 0.4) (layers F.Cu B.Cu) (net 14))
 (segment (start 69.85 109.22) (end 88.9 109.22) (width 0.25) (layer B.Cu) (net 14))
 (segment (start 69.85 109.22) (end 71.12 107.95) (width 0.25) (layer B.Cu) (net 14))
 (segment (start 71.12 107.95) (end 71.12 109.22) (width 0.25) (layer F.Cu) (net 14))
 (segment (start 70.35 109.99) (end 68.21 109.99) (width 0.25) (layer F.Cu) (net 14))
 (segment (start 71.12 109.22) (end 70.35 109.99) (width 0.25) (layer F.Cu) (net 14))
 (via (at 110.49 110.49) (size 0.8) (drill 0.4) (layers F.Cu B.Cu) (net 13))
 (segment (start 109.22 111.76) (end 110.49 110.49) (width 0.25) (layer B.Cu) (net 13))
 (segment (start 110.49 110.49) (end 109.22 111.76) (width 0.25) (layer F.Cu) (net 13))
 (segment (start 109.22 111.76) (end 107.95 111.76) (width 0.25) (layer F.Cu) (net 13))
 (segment (start 107.18 110.99) (end 106.31 110.99) (width 0.25) (layer F.Cu) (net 13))
 (segment (start 107.95 111.76) (end 107.18 110.99) (width 0.25) (layer F.Cu) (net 13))
 (via (at 91.44 110.49) (size 0.8) (drill 0.4) (layers F.Cu B.Cu) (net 13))
 (segment (start 90.17 111.76) (end 91.44 110.49) (width 0.25) (layer B.Cu) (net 13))
 (segment (start 90.17 111.76) (end 109.22 111.76) (width 0.25) (layer B.Cu) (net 13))
 (segment (start 91.44 110.49) (end 90.17 111.76) (width 0.25) (layer F.Cu) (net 13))
 (segment (start 90.17 111.76) (end 88.9 111.76) (width 0.25) (layer F.Cu) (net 13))
 (segment (start 88.13 110.99) (end 87.26 110.99) (width 0.25) (layer F.Cu) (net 13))
 (segment (start 88.9 111.76) (end 88.13 110.99) (width 0.25) (layer F.Cu) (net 13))
 (segment (start 71.12 111.76) (end 90.17 111.76) (width 0.25) (layer B.Cu) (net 13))
 (segment (start 71.12 111.76) (end 72.39 110.49) (width 0.25) (layer B.Cu) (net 13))
 (via (at 72.39 110.49) (size 0.8) (drill 0.4) (layers F.Cu B.Cu) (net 13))
 (segment (start 72.39 110.49) (end 71.12 111.76) (width 0.25) (layer F.Cu) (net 13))
 (segment (start 71.12 111.76) (end 69.85 111.76) (width 0.25) (layer F.Cu) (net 13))
 (segment (start 69.08 110.99) (end 68.21 110.99) (width 0.25) (layer F.Cu) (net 13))
 (segment (start 69.85 111.76) (end 69.08 110.99) (width 0.25) (layer F.Cu) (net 13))
 (segment (start 78.74 107.95) (end 82.55 107.95) (width 0.25) (layer F.Cu) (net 4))
 (segment (start 84.59 109.99) (end 85.46 109.99) (width 0.25) (layer F.Cu) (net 4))
 (segment (start 82.55 107.95) (end 84.59 109.99) (width 0.25) (layer F.Cu) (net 4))
 (segment (start 84.59 90.94) (end 85.46 90.94) (width 0.25) (layer F.Cu) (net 4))
 (segment (start 78.74 107.95) (end 78.74 88.9) (width 0.25) (layer F.Cu) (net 4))
 (segment (start 82.55 88.9) (end 84.59 90.94) (width 0.25) (layer F.Cu) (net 4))
 (segment (start 78.74 88.9) (end 82.55 88.9) (width 0.25) (layer F.Cu) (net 4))
 (segment (start 97.79 107.95) (end 101.6 107.95) (width 0.25) (layer F.Cu) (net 6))
 (segment (start 103.64 109.99) (end 104.51 109.99) (width 0.25) (layer F.Cu) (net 6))
 (segment (start 101.6 107.95) (end 103.64 109.99) (width 0.25) (layer F.Cu) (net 6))
 (segment (start 103.64 90.94) (end 104.51 90.94) (width 0.25) (layer F.Cu) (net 6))
 (segment (start 101.6 88.9) (end 103.64 90.94) (width 0.25) (layer F.Cu) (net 6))
 (segment (start 97.79 107.95) (end 97.79 88.9) (width 0.25) (layer F.Cu) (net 6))
 (segment (start 97.79 88.9) (end 101.6 88.9) (width 0.25) (layer F.Cu) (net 6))
 (via (at 71.12 91.44) (size 0.8) (drill 0.4) (layers F.Cu B.Cu) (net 10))
 (segment (start 91.44 92.71) (end 90.17 91.44) (width 0.25) (layer B.Cu) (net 10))
 (via (at 90.17 91.44) (size 0.8) (drill 0.4) (layers F.Cu B.Cu) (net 10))
 (segment (start 90.17 91.44) (end 88.9 91.44) (width 0.25) (layer F.Cu) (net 10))
 (segment (start 88.4 91.94) (end 87.26 91.94) (width 0.25) (layer F.Cu) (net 10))
 (segment (start 88.9 91.44) (end 88.4 91.94) (width 0.25) (layer F.Cu) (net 10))
 (via (at 109.22 91.44) (size 0.8) (drill 0.4) (layers F.Cu B.Cu) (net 10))
 (segment (start 110.49 92.71) (end 109.22 91.44) (width 0.25) (layer B.Cu) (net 10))
 (segment (start 110.49 92.71) (end 91.44 92.71) (width 0.25) (layer B.Cu) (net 10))
 (segment (start 109.22 91.44) (end 107.95 91.44) (width 0.25) (layer F.Cu) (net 10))
 (segment (start 107.45 91.94) (end 106.31 91.94) (width 0.25) (layer F.Cu) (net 10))
 (segment (start 107.95 91.44) (end 107.45 91.94) (width 0.25) (layer F.Cu) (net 10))
 (segment (start 91.44 92.71) (end 72.39 92.71) (width 0.25) (layer B.Cu) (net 10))
 (segment (start 72.39 92.71) (end 71.12 91.44) (width 0.25) (layer B.Cu) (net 10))
 (segment (start 71.12 91.44) (end 69.85 91.44) (width 0.25) (layer F.Cu) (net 10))
 (segment (start 69.35 91.94) (end 68.21 91.94) (width 0.25) (layer F.Cu) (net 10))
 (segment (start 69.85 91.44) (end 69.35 91.94) (width 0.25) (layer F.Cu) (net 10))
 (segment (start 116.040001 100.165001) (end 112.865001 100.165001) (width 0.25) (layer B.Cu) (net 10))
 (segment (start 116.84 100.965) (end 116.040001 100.165001) (width 0.25) (layer B.Cu) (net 10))
 (segment (start 112.865001 100.165001) (end 111.76 99.06) (width 0.25) (layer B.Cu) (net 10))
 (segment (start 111.76 99.06) (end 111.76 93.98) (width 0.25) (layer B.Cu) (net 10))
 (segment (start 111.76 93.98) (end 110.49 92.71) (width 0.25) (layer B.Cu) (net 10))
 (segment (start 111.76 90.17) (end 110.49 90.17) (width 0.25) (layer B.Cu) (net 11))
 (segment (start 115.70863 98.425) (end 115.07363 97.79) (width 0.25) (layer B.Cu) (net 11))
 (segment (start 116.84 98.425) (end 115.70863 98.425) (width 0.25) (layer B.Cu) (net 11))
 (segment (start 115.07363 97.79) (end 114.3 97.79) (width 0.25) (layer B.Cu) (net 11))
 (segment (start 114.3 97.79) (end 113.03 96.52) (width 0.25) (layer B.Cu) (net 11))
 (segment (start 113.03 91.44) (end 111.76 90.17) (width 0.25) (layer B.Cu) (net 11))
 (segment (start 113.03 96.52) (end 113.03 91.44) (width 0.25) (layer B.Cu) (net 11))
 (segment (start 59.69 107.95) (end 59.69 102.87) (width 0.25) (layer F.Cu) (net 2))
 (segment (start 55.88 98.425) (end 59.69 98.425) (width 0.25) (layer F.Cu) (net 2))
 (segment (start 59.69 102.87) (end 59.69 98.425) (width 0.25) (layer F.Cu) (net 2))
 (segment (start 59.69 98.425) (end 59.69 88.9) (width 0.25) (layer F.Cu) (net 2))
 (via (at 63.5 93.98) (size 0.8) (drill 0.4) (layers F.Cu B.Cu) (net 9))
 (segment (start 63.5 93.98) (end 63.5 92.71) (width 0.25) (layer F.Cu) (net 9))
 (segment (start 64.27 91.94) (end 66.41 91.94) (width 0.25) (layer F.Cu) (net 9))
 (segment (start 63.5 92.71) (end 64.27 91.94) (width 0.25) (layer F.Cu) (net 9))
 (segment (start 82.55 93.98) (end 63.5 93.98) (width 0.25) (layer B.Cu) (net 9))
 (via (at 82.55 93.98) (size 0.8) (drill 0.4) (layers F.Cu B.Cu) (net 9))
 (segment (start 82.55 93.98) (end 82.55 92.71) (width 0.25) (layer F.Cu) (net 9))
 (segment (start 83.32 91.94) (end 85.46 91.94) (width 0.25) (layer F.Cu) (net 9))
 (segment (start 82.55 92.71) (end 83.32 91.94) (width 0.25) (layer F.Cu) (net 9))
 (via (at 101.6 93.98) (size 0.8) (drill 0.4) (layers F.Cu B.Cu) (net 9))
 (segment (start 101.6 93.98) (end 82.55 93.98) (width 0.25) (layer B.Cu) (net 9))
 (segment (start 101.6 93.98) (end 101.6 92.71) (width 0.25) (layer F.Cu) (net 9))
 (segment (start 102.37 91.94) (end 104.51 91.94) (width 0.25) (layer F.Cu) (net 9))
 (segment (start 101.6 92.71) (end 102.37 91.94) (width 0.25) (layer F.Cu) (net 9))
 (segment (start 115.70863 103.505) (end 113.80363 101.6) (width 0.25) (layer B.Cu) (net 9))
 (segment (start 116.84 103.505) (end 115.70863 103.505) (width 0.25) (layer B.Cu) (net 9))
 (segment (start 113.80363 101.6) (end 111.76 101.6) (width 0.25) (layer B.Cu) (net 9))
 (segment (start 111.76 101.6) (end 110.49 100.33) (width 0.25) (layer B.Cu) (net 9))
 (segment (start 110.49 95.25) (end 109.22 93.98) (width 0.25) (layer B.Cu) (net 9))
 (segment (start 110.49 100.33) (end 110.49 95.25) (width 0.25) (layer B.Cu) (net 9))
 (segment (start 109.22 93.98) (end 101.6 93.98) (width 0.25) (layer B.Cu) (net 9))
 (segment (start 114.3 94.47637) (end 114.3 78.36) (width 0.25) (layer B.Cu) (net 7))
 (segment (start 115.70863 95.885) (end 114.3 94.47637) (width 0.25) (layer B.Cu) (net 7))
 (segment (start 114.3 78.36) (end 113.03 77.09) (width 0.25) (layer B.Cu) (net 7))
 (segment (start 116.84 95.885) (end 115.70863 95.885) (width 0.25) (layer B.Cu) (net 7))
 (segment (start 113.03 77.09) (end 101.6 77.09) (width 0.25) (layer B.Cu) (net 7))
 (segment (start 62.23 115.57) (end 64.77 115.57) (width 0.25) (layer B.Cu) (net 12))
 (segment (start 58.42 96.52) (end 58.42 111.76) (width 0.25) (layer B.Cu) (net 12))
 (segment (start 55.88 95.885) (end 57.785 95.885) (width 0.25) (layer B.Cu) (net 12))
 (segment (start 58.42 111.76) (end 62.23 115.57) (width 0.25) (layer B.Cu) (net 12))
 (segment (start 57.785 95.885) (end 58.42 96.52) (width 0.25) (layer B.Cu) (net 12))
 (segment (start 60.96 107.95) (end 62.23 109.22) (width 0.25) (layer B.Cu) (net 14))
 (segment (start 60.96 92.71) (end 60.96 107.95) (width 0.25) (layer B.Cu) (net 14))
 (segment (start 62.23 109.22) (end 69.85 109.22) (width 0.25) (layer B.Cu) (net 14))
 (segment (start 55.88 90.805) (end 59.055 90.805) (width 0.25) (layer B.Cu) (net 14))
 (segment (start 59.055 90.805) (end 60.96 92.71) (width 0.25) (layer B.Cu) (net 14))
 (segment (start 59.69 95.25) (end 59.69 109.22) (width 0.25) (layer B.Cu) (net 13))
 (segment (start 59.69 109.22) (end 62.23 111.76) (width 0.25) (layer B.Cu) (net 13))
 (segment (start 55.88 93.345) (end 57.785 93.345) (width 0.25) (layer B.Cu) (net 13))
 (segment (start 57.785 93.345) (end 59.69 95.25) (width 0.25) (layer B.Cu) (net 13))
 (segment (start 62.23 111.76) (end 71.12 111.76) (width 0.25) (layer B.Cu) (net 13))
 (segment (start 63.5 95.44) (end 63.5 96.14) (width 0.25) (layer B.Cu) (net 8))
 (segment (start 62.23 90.17) (end 62.23 94.17) (width 0.25) (layer B.Cu) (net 8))
 (segment (start 62.23 94.17) (end 63.5 95.44) (width 0.25) (layer B.Cu) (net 8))
 (segment (start 55.88 88.265) (end 60.325 88.265) (width 0.25) (layer B.Cu) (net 8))
 (segment (start 60.325 88.265) (end 62.23 90.17) (width 0.25) (layer B.Cu) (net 8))
 (segment (start 78.74 114.3) (end 77.47 115.57) (width 0.25) (layer F.Cu) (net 4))
 (segment (start 78.74 107.95) (end 78.74 114.3) (width 0.25) (layer F.Cu) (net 4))
 (segment (start 55.88 100.965) (end 57.785 100.965) (width 0.25) (layer F.Cu) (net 4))
 (segment (start 57.785 100.965) (end 58.42 101.6) (width 0.25) (layer F.Cu) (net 4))
 (segment (start 58.42 110.49) (end 63.5 115.57) (width 0.25) (layer F.Cu) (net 4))
 (segment (start 63.5 115.57) (end 77.47 115.57) (width 0.25) (layer F.Cu) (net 4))
 (segment (start 58.42 101.6) (end 58.42 110.49) (width 0.25) (layer F.Cu) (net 4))
 (segment (start 97.79 114.3) (end 95.25 116.84) (width 0.25) (layer F.Cu) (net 6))
 (segment (start 57.15 104.775) (end 55.88 103.505) (width 0.25) (layer F.Cu) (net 6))
 (segment (start 97.79 107.95) (end 97.79 114.3) (width 0.25) (layer F.Cu) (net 6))
 (segment (start 57.15 104.775) (end 57.15 111.76) (width 0.25) (layer F.Cu) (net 6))
 (segment (start 57.15 111.76) (end 62.23 116.84) (width 0.25) (layer F.Cu) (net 6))
 (segment (start 95.25 116.84) (end 62.23 116.84) (width 0.25) (layer F.Cu) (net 6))
 (segment (start 74.93 76.2) (end 72.39 78.74) (width 0.25) (layer F.Cu) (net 1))
 (segment (start 72.39 78.74) (end 72.39 80.01) (width 0.25) (layer F.Cu) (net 1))
 (segment (start 116.040001 87.465001) (end 114.464999 87.465001) (width 0.25) (layer F.Cu) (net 1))
 (segment (start 116.84 88.265) (end 116.040001 87.465001) (width 0.25) (layer F.Cu) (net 1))
 (segment (start 114.464999 87.465001) (end 113.359998 86.36) (width 0.25) (layer F.Cu) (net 1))
 (segment (start 113.359998 86.36) (end 113.359998 77.799998) (width 0.25) (layer F.Cu) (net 1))
 (segment (start 113.359998 77.799998) (end 111.76 76.2) (width 0.25) (layer F.Cu) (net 1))
 (segment (start 111.76 76.2) (end 74.93 76.2) (width 0.25) (layer F.Cu) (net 1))
 (segment (start 92.71 77.47) (end 91.44 78.74) (width 0.25) (layer F.Cu) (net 3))
 (segment (start 91.44 78.74) (end 91.44 80.01) (width 0.25) (layer F.Cu) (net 3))
 (segment (start 116.040001 90.005001) (end 113.194999 90.005001) (width 0.25) (layer F.Cu) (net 3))
 (segment (start 116.84 90.805) (end 116.040001 90.005001) (width 0.25) (layer F.Cu) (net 3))
 (segment (start 113.194999 90.005001) (end 111.76 88.570002) (width 0.25) (layer F.Cu) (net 3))
 (segment (start 111.76 88.570002) (end 111.76 78.74) (width 0.25) (layer F.Cu) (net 3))
 (segment (start 111.76 78.74) (end 110.49 77.47) (width 0.25) (layer F.Cu) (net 3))
 (segment (start 110.49 77.47) (end 92.71 77.47) (width 0.25) (layer F.Cu) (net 3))
 (segment (start 110.49 80.01) (end 110.49 81.28) (width 0.25) (layer F.Cu) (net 5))
 (segment (start 116.84 93.345) (end 116.040001 92.545001) (width 0.25) (layer F.Cu) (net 5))
 (segment (start 110.49 81.28) (end 110.49 90.17) (width 0.25) (layer F.Cu) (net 5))
 (segment (start 112.865001 92.545001) (end 110.49 90.17) (width 0.25) (layer F.Cu) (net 5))
 (segment (start 116.040001 92.545001) (end 112.865001 92.545001) (width 0.25) (layer F.Cu) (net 5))
 (segment (start 110.49 90.17) (end 110.49 99.06) (width 0.25) (layer F.Cu) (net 5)))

